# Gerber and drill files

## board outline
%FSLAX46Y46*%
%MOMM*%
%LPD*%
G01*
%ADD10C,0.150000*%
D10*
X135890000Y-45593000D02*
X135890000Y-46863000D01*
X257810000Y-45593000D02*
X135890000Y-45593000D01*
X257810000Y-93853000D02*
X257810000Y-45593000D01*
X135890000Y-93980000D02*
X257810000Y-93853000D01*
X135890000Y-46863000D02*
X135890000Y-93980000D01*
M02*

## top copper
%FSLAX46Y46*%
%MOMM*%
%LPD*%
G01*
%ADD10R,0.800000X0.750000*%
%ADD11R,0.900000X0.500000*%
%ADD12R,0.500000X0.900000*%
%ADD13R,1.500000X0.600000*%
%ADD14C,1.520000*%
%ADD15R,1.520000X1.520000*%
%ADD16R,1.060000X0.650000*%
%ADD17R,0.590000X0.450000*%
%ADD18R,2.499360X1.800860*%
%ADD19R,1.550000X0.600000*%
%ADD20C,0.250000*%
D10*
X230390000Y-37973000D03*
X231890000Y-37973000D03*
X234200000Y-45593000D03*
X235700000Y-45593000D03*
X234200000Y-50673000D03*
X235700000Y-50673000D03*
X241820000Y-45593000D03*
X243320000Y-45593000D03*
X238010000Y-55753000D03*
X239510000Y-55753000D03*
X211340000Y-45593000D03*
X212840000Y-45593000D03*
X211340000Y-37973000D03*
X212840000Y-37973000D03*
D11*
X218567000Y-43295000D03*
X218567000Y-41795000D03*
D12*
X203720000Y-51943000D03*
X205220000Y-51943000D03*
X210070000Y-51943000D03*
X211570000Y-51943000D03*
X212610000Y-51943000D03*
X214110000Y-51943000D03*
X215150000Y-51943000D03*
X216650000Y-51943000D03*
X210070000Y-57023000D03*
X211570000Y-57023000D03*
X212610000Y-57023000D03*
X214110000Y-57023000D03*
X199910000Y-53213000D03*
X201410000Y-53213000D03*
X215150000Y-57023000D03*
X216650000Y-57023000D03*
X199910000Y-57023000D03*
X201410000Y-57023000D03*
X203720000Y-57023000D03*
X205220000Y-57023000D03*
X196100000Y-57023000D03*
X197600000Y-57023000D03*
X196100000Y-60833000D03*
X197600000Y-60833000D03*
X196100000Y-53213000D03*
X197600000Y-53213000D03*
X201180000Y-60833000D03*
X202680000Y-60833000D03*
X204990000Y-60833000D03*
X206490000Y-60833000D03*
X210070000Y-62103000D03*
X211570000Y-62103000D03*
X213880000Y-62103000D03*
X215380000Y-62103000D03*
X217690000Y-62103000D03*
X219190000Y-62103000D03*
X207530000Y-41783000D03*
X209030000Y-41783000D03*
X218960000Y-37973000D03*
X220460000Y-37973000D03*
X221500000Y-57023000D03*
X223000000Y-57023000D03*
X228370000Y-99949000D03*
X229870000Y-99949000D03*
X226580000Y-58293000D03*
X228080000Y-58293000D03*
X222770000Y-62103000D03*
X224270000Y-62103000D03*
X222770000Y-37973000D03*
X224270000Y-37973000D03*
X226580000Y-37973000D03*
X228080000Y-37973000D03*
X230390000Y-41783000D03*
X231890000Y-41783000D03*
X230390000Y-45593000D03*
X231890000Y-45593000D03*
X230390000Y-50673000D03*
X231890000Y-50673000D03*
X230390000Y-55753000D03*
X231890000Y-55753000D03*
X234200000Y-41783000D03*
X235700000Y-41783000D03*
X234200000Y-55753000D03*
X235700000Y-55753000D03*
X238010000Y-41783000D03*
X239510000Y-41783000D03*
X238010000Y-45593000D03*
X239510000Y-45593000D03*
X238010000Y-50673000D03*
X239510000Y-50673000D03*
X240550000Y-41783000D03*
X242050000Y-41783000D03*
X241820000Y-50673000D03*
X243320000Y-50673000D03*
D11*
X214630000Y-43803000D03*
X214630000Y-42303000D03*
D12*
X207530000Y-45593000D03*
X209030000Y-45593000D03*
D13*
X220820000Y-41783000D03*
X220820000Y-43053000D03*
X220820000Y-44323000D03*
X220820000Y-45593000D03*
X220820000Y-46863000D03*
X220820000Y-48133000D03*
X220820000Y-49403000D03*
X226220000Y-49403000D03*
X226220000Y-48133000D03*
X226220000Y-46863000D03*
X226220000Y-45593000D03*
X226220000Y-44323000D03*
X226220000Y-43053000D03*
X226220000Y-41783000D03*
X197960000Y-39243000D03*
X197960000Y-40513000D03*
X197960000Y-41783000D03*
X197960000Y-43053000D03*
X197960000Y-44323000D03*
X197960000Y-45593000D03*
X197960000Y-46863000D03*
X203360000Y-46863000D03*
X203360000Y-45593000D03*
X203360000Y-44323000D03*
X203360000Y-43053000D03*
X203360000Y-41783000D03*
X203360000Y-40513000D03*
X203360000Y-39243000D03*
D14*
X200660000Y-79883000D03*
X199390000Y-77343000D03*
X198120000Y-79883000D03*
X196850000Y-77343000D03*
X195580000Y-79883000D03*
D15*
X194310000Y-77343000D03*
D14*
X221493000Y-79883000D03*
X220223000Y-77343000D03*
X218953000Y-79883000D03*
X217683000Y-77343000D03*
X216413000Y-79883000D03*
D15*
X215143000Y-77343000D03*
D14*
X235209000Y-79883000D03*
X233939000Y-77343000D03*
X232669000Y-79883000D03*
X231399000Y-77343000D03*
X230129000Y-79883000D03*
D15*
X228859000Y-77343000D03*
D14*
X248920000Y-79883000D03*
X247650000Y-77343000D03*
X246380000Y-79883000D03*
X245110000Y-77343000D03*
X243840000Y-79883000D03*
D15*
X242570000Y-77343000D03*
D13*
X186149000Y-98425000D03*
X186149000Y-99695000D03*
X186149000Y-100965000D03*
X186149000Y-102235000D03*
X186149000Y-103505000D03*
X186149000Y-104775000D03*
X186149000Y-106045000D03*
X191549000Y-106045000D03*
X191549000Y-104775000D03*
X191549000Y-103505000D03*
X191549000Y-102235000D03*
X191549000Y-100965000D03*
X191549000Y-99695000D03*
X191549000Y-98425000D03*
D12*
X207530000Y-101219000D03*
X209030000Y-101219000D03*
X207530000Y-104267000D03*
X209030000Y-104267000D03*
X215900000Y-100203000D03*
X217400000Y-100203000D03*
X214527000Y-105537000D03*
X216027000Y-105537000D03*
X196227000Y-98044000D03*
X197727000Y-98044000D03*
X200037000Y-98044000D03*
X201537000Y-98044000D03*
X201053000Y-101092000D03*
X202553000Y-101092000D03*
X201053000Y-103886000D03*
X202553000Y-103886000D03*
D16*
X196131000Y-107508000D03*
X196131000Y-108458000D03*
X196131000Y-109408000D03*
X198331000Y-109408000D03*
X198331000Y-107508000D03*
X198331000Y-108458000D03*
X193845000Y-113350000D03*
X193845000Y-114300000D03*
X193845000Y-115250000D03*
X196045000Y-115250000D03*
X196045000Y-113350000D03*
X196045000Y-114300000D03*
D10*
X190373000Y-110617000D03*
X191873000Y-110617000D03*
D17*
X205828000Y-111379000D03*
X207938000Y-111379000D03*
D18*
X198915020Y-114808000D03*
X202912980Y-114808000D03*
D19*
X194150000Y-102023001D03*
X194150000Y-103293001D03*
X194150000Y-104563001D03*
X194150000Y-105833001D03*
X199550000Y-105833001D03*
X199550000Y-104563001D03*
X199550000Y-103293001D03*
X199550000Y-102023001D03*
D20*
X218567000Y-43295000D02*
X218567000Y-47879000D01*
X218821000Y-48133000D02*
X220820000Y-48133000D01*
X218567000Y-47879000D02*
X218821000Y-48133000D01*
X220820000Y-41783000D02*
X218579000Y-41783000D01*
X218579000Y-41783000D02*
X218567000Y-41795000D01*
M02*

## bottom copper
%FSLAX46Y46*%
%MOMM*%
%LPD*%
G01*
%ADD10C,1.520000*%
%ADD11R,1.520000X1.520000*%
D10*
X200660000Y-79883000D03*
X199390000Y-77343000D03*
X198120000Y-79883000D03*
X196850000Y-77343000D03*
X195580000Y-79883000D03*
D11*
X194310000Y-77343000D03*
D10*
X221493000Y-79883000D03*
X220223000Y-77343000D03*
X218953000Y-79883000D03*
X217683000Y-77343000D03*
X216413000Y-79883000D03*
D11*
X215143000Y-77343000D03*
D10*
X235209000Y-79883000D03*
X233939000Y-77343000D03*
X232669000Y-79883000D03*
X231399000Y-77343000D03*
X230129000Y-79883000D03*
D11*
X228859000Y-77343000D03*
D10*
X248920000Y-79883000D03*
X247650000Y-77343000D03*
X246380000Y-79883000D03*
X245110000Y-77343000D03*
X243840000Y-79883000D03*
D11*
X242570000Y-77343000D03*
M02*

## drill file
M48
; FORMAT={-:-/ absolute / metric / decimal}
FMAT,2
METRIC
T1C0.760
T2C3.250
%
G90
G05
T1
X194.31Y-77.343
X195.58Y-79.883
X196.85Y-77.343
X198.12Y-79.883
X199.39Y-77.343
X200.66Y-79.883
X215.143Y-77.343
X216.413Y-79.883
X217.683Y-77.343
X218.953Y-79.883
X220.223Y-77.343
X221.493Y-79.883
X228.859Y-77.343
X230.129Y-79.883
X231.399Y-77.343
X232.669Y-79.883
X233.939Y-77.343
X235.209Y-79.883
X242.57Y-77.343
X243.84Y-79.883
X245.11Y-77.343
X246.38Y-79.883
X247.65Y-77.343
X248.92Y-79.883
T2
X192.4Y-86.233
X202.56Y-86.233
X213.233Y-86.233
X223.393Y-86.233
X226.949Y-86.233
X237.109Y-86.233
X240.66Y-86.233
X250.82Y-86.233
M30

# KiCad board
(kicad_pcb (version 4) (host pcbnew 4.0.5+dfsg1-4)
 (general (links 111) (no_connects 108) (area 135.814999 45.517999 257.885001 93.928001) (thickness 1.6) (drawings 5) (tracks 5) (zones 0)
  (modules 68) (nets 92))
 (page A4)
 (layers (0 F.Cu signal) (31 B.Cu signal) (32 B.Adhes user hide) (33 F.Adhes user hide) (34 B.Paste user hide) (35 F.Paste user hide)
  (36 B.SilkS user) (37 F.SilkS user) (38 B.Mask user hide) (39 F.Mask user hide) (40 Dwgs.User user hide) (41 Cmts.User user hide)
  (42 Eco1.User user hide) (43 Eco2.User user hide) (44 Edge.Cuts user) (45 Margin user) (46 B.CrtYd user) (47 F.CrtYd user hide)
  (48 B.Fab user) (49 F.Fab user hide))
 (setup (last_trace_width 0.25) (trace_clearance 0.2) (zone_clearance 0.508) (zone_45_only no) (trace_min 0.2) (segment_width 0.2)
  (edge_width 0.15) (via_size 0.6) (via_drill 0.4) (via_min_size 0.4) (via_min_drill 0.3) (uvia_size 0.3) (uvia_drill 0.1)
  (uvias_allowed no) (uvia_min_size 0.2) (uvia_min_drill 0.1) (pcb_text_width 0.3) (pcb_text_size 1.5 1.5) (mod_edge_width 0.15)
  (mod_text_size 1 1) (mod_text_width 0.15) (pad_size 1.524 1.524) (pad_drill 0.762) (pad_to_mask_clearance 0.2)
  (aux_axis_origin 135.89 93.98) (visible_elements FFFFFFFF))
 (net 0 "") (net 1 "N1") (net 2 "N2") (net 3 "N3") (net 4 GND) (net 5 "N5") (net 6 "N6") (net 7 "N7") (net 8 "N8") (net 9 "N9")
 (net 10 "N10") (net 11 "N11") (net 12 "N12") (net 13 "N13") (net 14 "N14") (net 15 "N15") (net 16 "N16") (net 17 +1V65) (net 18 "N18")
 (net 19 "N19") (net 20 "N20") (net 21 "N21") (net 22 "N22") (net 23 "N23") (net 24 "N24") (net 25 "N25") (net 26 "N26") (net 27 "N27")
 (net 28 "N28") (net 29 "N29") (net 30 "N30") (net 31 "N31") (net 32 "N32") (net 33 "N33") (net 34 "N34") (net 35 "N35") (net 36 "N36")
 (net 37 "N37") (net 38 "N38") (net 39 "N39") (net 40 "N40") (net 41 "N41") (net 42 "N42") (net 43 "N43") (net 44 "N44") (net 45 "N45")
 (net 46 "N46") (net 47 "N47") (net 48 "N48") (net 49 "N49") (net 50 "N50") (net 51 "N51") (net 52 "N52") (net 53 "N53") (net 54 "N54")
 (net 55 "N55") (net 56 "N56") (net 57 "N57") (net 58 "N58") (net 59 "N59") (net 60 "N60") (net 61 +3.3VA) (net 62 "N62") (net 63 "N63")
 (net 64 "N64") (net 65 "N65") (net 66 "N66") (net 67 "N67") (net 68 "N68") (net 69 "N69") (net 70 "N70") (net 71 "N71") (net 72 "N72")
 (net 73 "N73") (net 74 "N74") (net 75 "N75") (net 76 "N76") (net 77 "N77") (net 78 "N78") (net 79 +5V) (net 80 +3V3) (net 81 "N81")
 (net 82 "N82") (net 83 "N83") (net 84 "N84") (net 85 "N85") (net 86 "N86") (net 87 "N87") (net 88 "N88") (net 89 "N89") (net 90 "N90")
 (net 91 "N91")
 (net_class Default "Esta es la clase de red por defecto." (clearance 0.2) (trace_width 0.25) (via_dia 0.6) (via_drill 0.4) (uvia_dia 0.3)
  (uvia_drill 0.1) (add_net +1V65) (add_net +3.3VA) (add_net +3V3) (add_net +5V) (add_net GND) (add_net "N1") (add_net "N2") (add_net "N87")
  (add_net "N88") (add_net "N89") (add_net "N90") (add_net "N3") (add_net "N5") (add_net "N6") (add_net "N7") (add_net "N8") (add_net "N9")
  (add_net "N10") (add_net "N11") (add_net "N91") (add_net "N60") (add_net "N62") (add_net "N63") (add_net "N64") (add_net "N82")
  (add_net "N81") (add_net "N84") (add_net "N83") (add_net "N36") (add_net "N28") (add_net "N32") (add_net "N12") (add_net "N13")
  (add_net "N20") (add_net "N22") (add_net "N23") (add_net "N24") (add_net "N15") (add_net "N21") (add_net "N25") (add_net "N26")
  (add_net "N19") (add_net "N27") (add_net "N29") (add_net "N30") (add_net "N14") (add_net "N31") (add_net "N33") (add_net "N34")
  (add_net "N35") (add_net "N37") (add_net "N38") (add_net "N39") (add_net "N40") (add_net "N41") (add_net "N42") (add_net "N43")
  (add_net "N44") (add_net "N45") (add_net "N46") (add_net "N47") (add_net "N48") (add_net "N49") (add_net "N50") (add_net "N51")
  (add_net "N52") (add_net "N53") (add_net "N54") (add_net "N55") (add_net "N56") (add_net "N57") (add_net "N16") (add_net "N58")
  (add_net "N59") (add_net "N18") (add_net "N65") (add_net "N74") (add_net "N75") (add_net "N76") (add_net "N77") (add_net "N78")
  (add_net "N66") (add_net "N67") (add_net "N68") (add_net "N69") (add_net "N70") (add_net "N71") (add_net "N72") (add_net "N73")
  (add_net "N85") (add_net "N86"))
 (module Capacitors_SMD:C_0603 (layer F.Cu) (at 231.14 37.973)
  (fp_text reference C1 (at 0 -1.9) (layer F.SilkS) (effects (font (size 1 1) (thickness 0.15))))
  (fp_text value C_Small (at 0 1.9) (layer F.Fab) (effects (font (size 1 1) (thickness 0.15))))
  (pad 1 smd rect (at -0.75 0) (size 0.8 0.75) (layers F.Cu F.Paste F.Mask) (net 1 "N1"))
  (pad 2 smd rect (at 0.75 0) (size 0.8 0.75) (layers F.Cu F.Paste F.Mask) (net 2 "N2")))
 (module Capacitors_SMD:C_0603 (layer F.Cu) (at 234.95 45.593)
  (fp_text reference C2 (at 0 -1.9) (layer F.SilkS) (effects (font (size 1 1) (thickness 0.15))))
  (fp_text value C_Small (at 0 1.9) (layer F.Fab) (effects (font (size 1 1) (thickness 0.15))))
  (pad 1 smd rect (at -0.75 0) (size 0.8 0.75) (layers F.Cu F.Paste F.Mask) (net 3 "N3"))
  (pad 2 smd rect (at 0.75 0) (size 0.8 0.75) (layers F.Cu F.Paste F.Mask) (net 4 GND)))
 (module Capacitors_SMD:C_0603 (layer F.Cu) (at 234.95 50.673)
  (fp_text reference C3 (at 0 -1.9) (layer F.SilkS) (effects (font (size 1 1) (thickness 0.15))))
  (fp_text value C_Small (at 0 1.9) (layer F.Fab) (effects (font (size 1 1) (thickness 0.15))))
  (pad 1 smd rect (at -0.75 0) (size 0.8 0.75) (layers F.Cu F.Paste F.Mask) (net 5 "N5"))
  (pad 2 smd rect (at 0.75 0) (size 0.8 0.75) (layers F.Cu F.Paste F.Mask) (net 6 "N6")))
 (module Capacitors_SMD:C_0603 (layer F.Cu) (at 242.57 45.593)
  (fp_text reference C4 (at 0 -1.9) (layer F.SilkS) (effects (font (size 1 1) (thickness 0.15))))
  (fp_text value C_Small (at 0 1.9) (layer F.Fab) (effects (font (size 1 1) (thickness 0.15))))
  (pad 1 smd rect (at -0.75 0) (size 0.8 0.75) (layers F.Cu F.Paste F.Mask) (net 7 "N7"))
  (pad 2 smd rect (at 0.75 0) (size 0.8 0.75) (layers F.Cu F.Paste F.Mask) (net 4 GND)))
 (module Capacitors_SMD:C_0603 (layer F.Cu) (at 238.76 55.753)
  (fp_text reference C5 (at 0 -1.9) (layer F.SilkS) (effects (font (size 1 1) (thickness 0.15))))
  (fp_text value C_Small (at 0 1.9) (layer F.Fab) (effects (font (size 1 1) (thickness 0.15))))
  (pad 1 smd rect (at -0.75 0) (size 0.8 0.75) (layers F.Cu F.Paste F.Mask) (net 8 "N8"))
  (pad 2 smd rect (at 0.75 0) (size 0.8 0.75) (layers F.Cu F.Paste F.Mask) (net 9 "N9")))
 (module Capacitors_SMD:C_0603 (layer F.Cu) (at 212.09 45.593)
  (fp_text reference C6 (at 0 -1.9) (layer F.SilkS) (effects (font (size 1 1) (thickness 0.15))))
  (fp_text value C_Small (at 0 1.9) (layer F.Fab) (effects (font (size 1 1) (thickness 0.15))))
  (pad 1 smd rect (at -0.75 0) (size 0.8 0.75) (layers F.Cu F.Paste F.Mask) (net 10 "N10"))
  (pad 2 smd rect (at 0.75 0) (size 0.8 0.75) (layers F.Cu F.Paste F.Mask) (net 4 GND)))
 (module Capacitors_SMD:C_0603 (layer F.Cu) (at 212.09 37.973)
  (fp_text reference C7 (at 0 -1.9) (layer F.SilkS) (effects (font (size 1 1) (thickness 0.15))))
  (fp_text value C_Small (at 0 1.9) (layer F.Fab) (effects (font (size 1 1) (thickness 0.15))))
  (pad 1 smd rect (at -0.75 0) (size 0.8 0.75) (layers F.Cu F.Paste F.Mask) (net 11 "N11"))
  (pad 2 smd rect (at 0.75 0) (size 0.8 0.75) (layers F.Cu F.Paste F.Mask) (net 4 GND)))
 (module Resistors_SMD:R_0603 (layer F.Cu) (at 218.567 42.545 90)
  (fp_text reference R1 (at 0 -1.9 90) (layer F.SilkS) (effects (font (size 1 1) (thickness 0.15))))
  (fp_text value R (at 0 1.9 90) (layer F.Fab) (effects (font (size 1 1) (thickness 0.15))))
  (pad 1 smd rect (at -0.75 0 90) (size 0.5 0.9) (layers F.Cu F.Paste F.Mask) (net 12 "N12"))
  (pad 2 smd rect (at 0.75 0 90) (size 0.5 0.9) (layers F.Cu F.Paste F.Mask) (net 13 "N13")))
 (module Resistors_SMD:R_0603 (layer F.Cu) (at 204.47 51.943)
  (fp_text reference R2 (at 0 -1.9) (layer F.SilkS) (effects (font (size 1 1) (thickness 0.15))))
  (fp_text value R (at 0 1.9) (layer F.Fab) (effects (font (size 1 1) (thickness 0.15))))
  (pad 1 smd rect (at -0.75 0) (size 0.5 0.9) (layers F.Cu F.Paste F.Mask) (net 13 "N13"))
  (pad 2 smd rect (at 0.75 0) (size 0.5 0.9) (layers F.Cu F.Paste F.Mask) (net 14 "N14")))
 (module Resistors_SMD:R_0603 (layer F.Cu) (at 210.82 51.943)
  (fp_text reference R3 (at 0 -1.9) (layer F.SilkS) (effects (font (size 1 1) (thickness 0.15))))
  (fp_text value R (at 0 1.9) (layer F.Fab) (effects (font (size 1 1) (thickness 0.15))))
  (pad 1 smd rect (at -0.75 0) (size 0.5 0.9) (layers F.Cu F.Paste F.Mask) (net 7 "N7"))
  (pad 2 smd rect (at 0.75 0) (size 0.5 0.9) (layers F.Cu F.Paste F.Mask) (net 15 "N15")))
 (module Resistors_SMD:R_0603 (layer F.Cu) (at 213.36 51.943)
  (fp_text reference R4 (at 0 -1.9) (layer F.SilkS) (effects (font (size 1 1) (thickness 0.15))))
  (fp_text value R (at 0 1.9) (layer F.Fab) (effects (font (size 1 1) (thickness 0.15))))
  (pad 1 smd rect (at -0.75 0) (size 0.5 0.9) (layers F.Cu F.Paste F.Mask) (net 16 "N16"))
  (pad 2 smd rect (at 0.75 0) (size 0.5 0.9) (layers F.Cu F.Paste F.Mask) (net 12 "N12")))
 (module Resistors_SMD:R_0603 (layer F.Cu) (at 215.9 51.943)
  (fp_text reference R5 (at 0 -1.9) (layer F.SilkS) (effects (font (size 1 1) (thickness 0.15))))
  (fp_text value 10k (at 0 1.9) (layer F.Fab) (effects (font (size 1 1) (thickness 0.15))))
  (pad 1 smd rect (at -0.75 0) (size 0.5 0.9) (layers F.Cu F.Paste F.Mask) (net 14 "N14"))
  (pad 2 smd rect (at 0.75 0) (size 0.5 0.9) (layers F.Cu F.Paste F.Mask) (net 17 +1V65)))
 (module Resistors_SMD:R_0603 (layer F.Cu) (at 210.82 57.023)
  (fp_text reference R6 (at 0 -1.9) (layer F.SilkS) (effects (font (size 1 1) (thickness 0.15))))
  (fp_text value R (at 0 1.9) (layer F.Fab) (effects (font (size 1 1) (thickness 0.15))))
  (pad 1 smd rect (at -0.75 0) (size 0.5 0.9) (layers F.Cu F.Paste F.Mask) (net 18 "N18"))
  (pad 2 smd rect (at 0.75 0) (size 0.5 0.9) (layers F.Cu F.Paste F.Mask) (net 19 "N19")))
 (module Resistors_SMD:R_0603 (layer F.Cu) (at 213.36 57.023)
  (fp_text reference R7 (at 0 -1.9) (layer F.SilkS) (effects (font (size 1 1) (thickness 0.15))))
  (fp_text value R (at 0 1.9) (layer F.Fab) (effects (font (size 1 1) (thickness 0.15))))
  (pad 1 smd rect (at -0.75 0) (size 0.5 0.9) (layers F.Cu F.Paste F.Mask) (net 3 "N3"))
  (pad 2 smd rect (at 0.75 0) (size 0.5 0.9) (layers F.Cu F.Paste F.Mask) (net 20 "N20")))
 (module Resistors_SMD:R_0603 (layer F.Cu) (at 200.66 53.213)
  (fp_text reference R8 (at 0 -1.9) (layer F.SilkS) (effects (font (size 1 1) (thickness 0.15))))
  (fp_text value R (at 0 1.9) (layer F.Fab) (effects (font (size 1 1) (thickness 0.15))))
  (pad 1 smd rect (at -0.75 0) (size 0.5 0.9) (layers F.Cu F.Paste F.Mask) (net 10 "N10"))
  (pad 2 smd rect (at 0.75 0) (size 0.5 0.9) (layers F.Cu F.Paste F.Mask) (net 16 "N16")))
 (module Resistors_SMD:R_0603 (layer F.Cu) (at 215.9 57.023)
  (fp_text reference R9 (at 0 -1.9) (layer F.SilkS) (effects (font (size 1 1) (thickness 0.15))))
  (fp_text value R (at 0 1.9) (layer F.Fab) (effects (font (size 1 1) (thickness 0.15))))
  (pad 1 smd rect (at -0.75 0) (size 0.5 0.9) (layers F.Cu F.Paste F.Mask) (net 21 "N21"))
  (pad 2 smd rect (at 0.75 0) (size 0.5 0.9) (layers F.Cu F.Paste F.Mask) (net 18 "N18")))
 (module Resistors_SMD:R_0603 (layer F.Cu) (at 200.66 57.023)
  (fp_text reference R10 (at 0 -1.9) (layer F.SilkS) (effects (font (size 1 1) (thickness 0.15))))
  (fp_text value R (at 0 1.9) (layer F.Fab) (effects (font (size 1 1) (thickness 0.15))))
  (pad 1 smd rect (at -0.75 0) (size 0.5 0.9) (layers F.Cu F.Paste F.Mask) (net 20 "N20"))
  (pad 2 smd rect (at 0.75 0) (size 0.5 0.9) (layers F.Cu F.Paste F.Mask) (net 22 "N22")))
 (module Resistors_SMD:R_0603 (layer F.Cu) (at 204.47 57.023)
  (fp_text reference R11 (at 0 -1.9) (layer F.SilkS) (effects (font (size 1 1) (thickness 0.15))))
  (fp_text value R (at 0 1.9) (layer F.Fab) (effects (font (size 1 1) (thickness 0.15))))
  (pad 1 smd rect (at -0.75 0) (size 0.5 0.9) (layers F.Cu F.Paste F.Mask) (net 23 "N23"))
  (pad 2 smd rect (at 0.75 0) (size 0.5 0.9) (layers F.Cu F.Paste F.Mask) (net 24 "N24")))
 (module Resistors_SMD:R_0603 (layer F.Cu) (at 196.85 57.023)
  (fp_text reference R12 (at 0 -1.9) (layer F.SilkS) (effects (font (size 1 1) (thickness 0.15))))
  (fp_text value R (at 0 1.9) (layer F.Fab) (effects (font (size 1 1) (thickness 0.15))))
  (pad 1 smd rect (at -0.75 0) (size 0.5 0.9) (layers F.Cu F.Paste F.Mask) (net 15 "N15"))
  (pad 2 smd rect (at 0.75 0) (size 0.5 0.9) (layers F.Cu F.Paste F.Mask) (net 21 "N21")))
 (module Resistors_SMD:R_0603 (layer F.Cu) (at 196.85 60.833)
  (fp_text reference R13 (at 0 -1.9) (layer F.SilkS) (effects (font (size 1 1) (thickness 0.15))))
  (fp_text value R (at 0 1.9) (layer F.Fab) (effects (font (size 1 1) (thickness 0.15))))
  (pad 1 smd rect (at -0.75 0) (size 0.5 0.9) (layers F.Cu F.Paste F.Mask) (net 22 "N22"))
  (pad 2 smd rect (at 0.75 0) (size 0.5 0.9) (layers F.Cu F.Paste F.Mask) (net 23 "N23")))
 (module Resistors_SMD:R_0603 (layer F.Cu) (at 196.85 53.213)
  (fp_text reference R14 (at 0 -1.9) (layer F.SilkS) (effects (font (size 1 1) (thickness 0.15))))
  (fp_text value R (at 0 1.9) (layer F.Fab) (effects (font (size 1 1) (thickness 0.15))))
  (pad 1 smd rect (at -0.75 0) (size 0.5 0.9) (layers F.Cu F.Paste F.Mask) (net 11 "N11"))
  (pad 2 smd rect (at 0.75 0) (size 0.5 0.9) (layers F.Cu F.Paste F.Mask) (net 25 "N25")))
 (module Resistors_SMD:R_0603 (layer F.Cu) (at 201.93 60.833)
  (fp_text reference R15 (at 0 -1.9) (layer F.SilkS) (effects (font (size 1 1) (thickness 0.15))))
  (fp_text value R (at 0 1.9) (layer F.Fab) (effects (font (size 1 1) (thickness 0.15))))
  (pad 1 smd rect (at -0.75 0) (size 0.5 0.9) (layers F.Cu F.Paste F.Mask) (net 25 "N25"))
  (pad 2 smd rect (at 0.75 0) (size 0.5 0.9) (layers F.Cu F.Paste F.Mask) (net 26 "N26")))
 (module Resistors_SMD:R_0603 (layer F.Cu) (at 205.74 60.833)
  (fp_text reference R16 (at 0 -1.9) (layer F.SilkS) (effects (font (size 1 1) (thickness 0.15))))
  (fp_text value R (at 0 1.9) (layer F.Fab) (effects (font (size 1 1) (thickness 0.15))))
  (pad 1 smd rect (at -0.75 0) (size 0.5 0.9) (layers F.Cu F.Paste F.Mask) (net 19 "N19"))
  (pad 2 smd rect (at 0.75 0) (size 0.5 0.9) (layers F.Cu F.Paste F.Mask) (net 17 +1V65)))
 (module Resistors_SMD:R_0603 (layer F.Cu) (at 210.82 62.103)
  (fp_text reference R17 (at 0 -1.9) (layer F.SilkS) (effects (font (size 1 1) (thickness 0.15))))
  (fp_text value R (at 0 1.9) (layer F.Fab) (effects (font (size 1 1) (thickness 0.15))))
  (pad 1 smd rect (at -0.75 0) (size 0.5 0.9) (layers F.Cu F.Paste F.Mask) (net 24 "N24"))
  (pad 2 smd rect (at 0.75 0) (size 0.5 0.9) (layers F.Cu F.Paste F.Mask) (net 17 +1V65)))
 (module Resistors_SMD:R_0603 (layer F.Cu) (at 214.63 62.103)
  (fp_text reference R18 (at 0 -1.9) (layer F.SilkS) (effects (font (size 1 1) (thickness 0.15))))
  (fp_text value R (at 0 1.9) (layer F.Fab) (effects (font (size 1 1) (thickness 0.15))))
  (pad 1 smd rect (at -0.75 0) (size 0.5 0.9) (layers F.Cu F.Paste F.Mask) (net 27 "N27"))
  (pad 2 smd rect (at 0.75 0) (size 0.5 0.9) (layers F.Cu F.Paste F.Mask) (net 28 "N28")))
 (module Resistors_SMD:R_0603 (layer F.Cu) (at 218.44 62.103)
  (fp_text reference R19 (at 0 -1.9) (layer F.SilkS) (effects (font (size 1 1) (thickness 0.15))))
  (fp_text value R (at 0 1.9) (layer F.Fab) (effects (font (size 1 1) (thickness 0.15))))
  (pad 1 smd rect (at -0.75 0) (size 0.5 0.9) (layers F.Cu F.Paste F.Mask) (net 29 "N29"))
  (pad 2 smd rect (at 0.75 0) (size 0.5 0.9) (layers F.Cu F.Paste F.Mask) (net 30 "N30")))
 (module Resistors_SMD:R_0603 (layer F.Cu) (at 208.28 41.783)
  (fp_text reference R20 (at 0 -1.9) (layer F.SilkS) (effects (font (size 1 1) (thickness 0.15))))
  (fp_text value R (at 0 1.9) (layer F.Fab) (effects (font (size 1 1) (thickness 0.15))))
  (pad 1 smd rect (at -0.75 0) (size 0.5 0.9) (layers F.Cu F.Paste F.Mask) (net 26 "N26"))
  (pad 2 smd rect (at 0.75 0) (size 0.5 0.9) (layers F.Cu F.Paste F.Mask) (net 29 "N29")))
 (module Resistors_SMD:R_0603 (layer F.Cu) (at 219.71 37.973)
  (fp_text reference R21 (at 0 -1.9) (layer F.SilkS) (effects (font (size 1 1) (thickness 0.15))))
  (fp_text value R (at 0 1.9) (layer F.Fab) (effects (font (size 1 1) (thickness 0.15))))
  (pad 1 smd rect (at -0.75 0) (size 0.5 0.9) (layers F.Cu F.Paste F.Mask) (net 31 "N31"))
  (pad 2 smd rect (at 0.75 0) (size 0.5 0.9) (layers F.Cu F.Paste F.Mask) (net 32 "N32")))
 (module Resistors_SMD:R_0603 (layer F.Cu) (at 222.25 57.023)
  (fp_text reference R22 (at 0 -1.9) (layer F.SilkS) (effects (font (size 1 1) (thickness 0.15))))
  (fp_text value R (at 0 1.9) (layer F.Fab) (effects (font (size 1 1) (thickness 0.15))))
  (pad 1 smd rect (at -0.75 0) (size 0.5 0.9) (layers F.Cu F.Paste F.Mask) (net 30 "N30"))
  (pad 2 smd rect (at 0.75 0) (size 0.5 0.9) (layers F.Cu F.Paste F.Mask) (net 17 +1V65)))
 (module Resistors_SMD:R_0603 (layer F.Cu) (at 229.12 99.949)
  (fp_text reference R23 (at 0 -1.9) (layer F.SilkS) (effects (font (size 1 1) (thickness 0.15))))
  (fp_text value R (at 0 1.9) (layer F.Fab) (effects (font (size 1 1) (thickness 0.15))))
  (pad 1 smd rect (at -0.75 0) (size 0.5 0.9) (layers F.Cu F.Paste F.Mask) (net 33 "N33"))
  (pad 2 smd rect (at 0.75 0) (size 0.5 0.9) (layers F.Cu F.Paste F.Mask) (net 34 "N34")))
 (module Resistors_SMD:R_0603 (layer F.Cu) (at 227.33 58.293)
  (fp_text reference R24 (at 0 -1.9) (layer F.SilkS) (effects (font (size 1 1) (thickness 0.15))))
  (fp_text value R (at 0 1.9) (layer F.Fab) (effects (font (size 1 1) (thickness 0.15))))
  (pad 1 smd rect (at -0.75 0) (size 0.5 0.9) (layers F.Cu F.Paste F.Mask) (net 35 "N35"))
  (pad 2 smd rect (at 0.75 0) (size 0.5 0.9) (layers F.Cu F.Paste F.Mask) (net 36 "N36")))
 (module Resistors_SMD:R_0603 (layer F.Cu) (at 223.52 62.103)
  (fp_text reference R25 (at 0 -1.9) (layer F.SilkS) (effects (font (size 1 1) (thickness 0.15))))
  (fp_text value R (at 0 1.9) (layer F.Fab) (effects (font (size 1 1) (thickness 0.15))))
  (pad 1 smd rect (at -0.75 0) (size 0.5 0.9) (layers F.Cu F.Paste F.Mask) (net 35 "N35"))
  (pad 2 smd rect (at 0.75 0) (size 0.5 0.9) (layers F.Cu F.Paste F.Mask) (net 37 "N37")))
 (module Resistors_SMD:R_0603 (layer F.Cu) (at 223.52 37.973)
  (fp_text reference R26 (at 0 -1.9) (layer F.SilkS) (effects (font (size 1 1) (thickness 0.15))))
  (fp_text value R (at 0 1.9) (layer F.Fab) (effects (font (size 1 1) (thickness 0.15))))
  (pad 1 smd rect (at -0.75 0) (size 0.5 0.9) (layers F.Cu F.Paste F.Mask) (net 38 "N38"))
  (pad 2 smd rect (at 0.75 0) (size 0.5 0.9) (layers F.Cu F.Paste F.Mask) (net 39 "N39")))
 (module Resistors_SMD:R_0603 (layer F.Cu) (at 227.33 37.973)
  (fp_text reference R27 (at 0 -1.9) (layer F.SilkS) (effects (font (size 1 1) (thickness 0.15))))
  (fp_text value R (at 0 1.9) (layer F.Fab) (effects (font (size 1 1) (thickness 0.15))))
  (pad 1 smd rect (at -0.75 0) (size 0.5 0.9) (layers F.Cu F.Paste F.Mask) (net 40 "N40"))
  (pad 2 smd rect (at 0.75 0) (size 0.5 0.9) (layers F.Cu F.Paste F.Mask) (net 27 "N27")))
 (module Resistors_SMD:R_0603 (layer F.Cu) (at 231.14 41.783)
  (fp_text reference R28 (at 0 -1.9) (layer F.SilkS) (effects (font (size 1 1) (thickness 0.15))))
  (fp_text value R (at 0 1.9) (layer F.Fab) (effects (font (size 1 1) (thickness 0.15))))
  (pad 1 smd rect (at -0.75 0) (size 0.5 0.9) (layers F.Cu F.Paste F.Mask) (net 39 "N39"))
  (pad 2 smd rect (at 0.75 0) (size 0.5 0.9) (layers F.Cu F.Paste F.Mask) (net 31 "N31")))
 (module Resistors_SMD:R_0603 (layer F.Cu) (at 231.14 45.593)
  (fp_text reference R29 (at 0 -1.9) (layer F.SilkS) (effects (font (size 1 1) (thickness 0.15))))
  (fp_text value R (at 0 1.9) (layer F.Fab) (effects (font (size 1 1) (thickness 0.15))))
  (pad 1 smd rect (at -0.75 0) (size 0.5 0.9) (layers F.Cu F.Paste F.Mask) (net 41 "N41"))
  (pad 2 smd rect (at 0.75 0) (size 0.5 0.9) (layers F.Cu F.Paste F.Mask) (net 37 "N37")))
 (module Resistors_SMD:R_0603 (layer F.Cu) (at 231.14 50.673)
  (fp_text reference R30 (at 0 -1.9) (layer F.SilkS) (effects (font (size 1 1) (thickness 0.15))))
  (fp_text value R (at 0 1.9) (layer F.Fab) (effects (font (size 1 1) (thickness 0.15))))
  (pad 1 smd rect (at -0.75 0) (size 0.5 0.9) (layers F.Cu F.Paste F.Mask) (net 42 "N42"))
  (pad 2 smd rect (at 0.75 0) (size 0.5 0.9) (layers F.Cu F.Paste F.Mask) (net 40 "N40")))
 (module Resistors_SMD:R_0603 (layer F.Cu) (at 231.14 55.753)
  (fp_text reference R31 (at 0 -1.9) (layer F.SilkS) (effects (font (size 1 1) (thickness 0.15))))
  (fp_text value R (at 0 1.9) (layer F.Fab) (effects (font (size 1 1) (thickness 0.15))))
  (pad 1 smd rect (at -0.75 0) (size 0.5 0.9) (layers F.Cu F.Paste F.Mask) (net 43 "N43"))
  (pad 2 smd rect (at 0.75 0) (size 0.5 0.9) (layers F.Cu F.Paste F.Mask) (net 41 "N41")))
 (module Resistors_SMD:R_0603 (layer F.Cu) (at 234.95 41.783)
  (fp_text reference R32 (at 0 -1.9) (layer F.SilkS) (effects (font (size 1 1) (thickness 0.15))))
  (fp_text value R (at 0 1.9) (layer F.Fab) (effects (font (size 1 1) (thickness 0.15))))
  (pad 1 smd rect (at -0.75 0) (size 0.5 0.9) (layers F.Cu F.Paste F.Mask) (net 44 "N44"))
  (pad 2 smd rect (at 0.75 0) (size 0.5 0.9) (layers F.Cu F.Paste F.Mask) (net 42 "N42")))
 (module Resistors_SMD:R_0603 (layer F.Cu) (at 234.95 55.753)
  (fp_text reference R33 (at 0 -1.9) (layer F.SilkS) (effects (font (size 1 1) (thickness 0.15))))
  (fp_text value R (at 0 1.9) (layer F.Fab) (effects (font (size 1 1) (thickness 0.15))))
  (pad 1 smd rect (at -0.75 0) (size 0.5 0.9) (layers F.Cu F.Paste F.Mask) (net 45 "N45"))
  (pad 2 smd rect (at 0.75 0) (size 0.5 0.9) (layers F.Cu F.Paste F.Mask) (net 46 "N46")))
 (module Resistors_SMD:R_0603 (layer F.Cu) (at 238.76 41.783)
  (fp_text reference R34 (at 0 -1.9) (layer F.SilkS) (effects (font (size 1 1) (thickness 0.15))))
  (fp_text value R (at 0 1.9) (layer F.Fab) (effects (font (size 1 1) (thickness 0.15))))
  (pad 1 smd rect (at -0.75 0) (size 0.5 0.9) (layers F.Cu F.Paste F.Mask) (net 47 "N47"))
  (pad 2 smd rect (at 0.75 0) (size 0.5 0.9) (layers F.Cu F.Paste F.Mask) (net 38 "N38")))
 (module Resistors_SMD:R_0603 (layer F.Cu) (at 238.76 45.593)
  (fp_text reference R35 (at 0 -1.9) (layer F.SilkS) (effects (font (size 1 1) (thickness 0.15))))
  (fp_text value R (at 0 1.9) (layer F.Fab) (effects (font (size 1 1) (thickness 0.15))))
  (pad 1 smd rect (at -0.75 0) (size 0.5 0.9) (layers F.Cu F.Paste F.Mask) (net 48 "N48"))
  (pad 2 smd rect (at 0.75 0) (size 0.5 0.9) (layers F.Cu F.Paste F.Mask) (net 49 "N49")))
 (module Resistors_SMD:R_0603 (layer F.Cu) (at 238.76 50.673)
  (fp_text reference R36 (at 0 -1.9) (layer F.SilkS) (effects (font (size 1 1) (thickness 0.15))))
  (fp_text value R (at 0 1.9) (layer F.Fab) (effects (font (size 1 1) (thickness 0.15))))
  (pad 1 smd rect (at -0.75 0) (size 0.5 0.9) (layers F.Cu F.Paste F.Mask) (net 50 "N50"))
  (pad 2 smd rect (at 0.75 0) (size 0.5 0.9) (layers F.Cu F.Paste F.Mask) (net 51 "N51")))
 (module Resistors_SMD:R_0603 (layer F.Cu) (at 241.3 41.783)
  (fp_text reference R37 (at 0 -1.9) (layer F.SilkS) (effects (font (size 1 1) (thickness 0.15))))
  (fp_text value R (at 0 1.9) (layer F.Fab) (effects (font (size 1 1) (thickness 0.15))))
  (pad 1 smd rect (at -0.75 0) (size 0.5 0.9) (layers F.Cu F.Paste F.Mask) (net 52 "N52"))
  (pad 2 smd rect (at 0.75 0) (size 0.5 0.9) (layers F.Cu F.Paste F.Mask) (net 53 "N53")))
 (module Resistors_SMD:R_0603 (layer F.Cu) (at 242.57 50.673)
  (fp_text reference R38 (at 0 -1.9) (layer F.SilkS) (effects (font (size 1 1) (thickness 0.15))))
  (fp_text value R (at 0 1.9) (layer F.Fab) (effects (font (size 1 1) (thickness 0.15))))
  (pad 1 smd rect (at -0.75 0) (size 0.5 0.9) (layers F.Cu F.Paste F.Mask) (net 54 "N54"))
  (pad 2 smd rect (at 0.75 0) (size 0.5 0.9) (layers F.Cu F.Paste F.Mask) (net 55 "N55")))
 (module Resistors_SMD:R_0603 (layer F.Cu) (at 214.63 43.053 90)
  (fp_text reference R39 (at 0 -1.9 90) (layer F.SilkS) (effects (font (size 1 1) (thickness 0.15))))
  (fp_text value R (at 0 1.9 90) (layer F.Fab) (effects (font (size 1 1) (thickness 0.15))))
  (pad 1 smd rect (at -0.75 0 90) (size 0.5 0.9) (layers F.Cu F.Paste F.Mask) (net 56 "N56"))
  (pad 2 smd rect (at 0.75 0 90) (size 0.5 0.9) (layers F.Cu F.Paste F.Mask) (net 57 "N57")))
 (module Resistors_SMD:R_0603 (layer F.Cu) (at 208.28 45.593)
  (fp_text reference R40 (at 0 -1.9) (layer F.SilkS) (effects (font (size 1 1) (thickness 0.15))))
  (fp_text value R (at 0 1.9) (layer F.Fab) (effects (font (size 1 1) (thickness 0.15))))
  (pad 1 smd rect (at -0.75 0) (size 0.5 0.9) (layers F.Cu F.Paste F.Mask) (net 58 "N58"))
  (pad 2 smd rect (at 0.75 0) (size 0.5 0.9) (layers F.Cu F.Paste F.Mask) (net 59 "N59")))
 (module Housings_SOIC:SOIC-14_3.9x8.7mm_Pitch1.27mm (layer F.Cu) (at 223.52 45.593)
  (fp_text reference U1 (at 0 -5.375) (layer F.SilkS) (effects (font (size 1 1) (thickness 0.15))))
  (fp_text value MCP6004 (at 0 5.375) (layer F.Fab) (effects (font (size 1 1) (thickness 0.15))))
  (pad 1 smd rect (at -2.7 -3.81) (size 1.5 0.6) (layers F.Cu F.Paste F.Mask) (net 13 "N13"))
  (pad 2 smd rect (at -2.7 -2.54) (size 1.5 0.6) (layers F.Cu F.Paste F.Mask) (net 14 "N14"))
  (pad 3 smd rect (at -2.7 -1.27) (size 1.5 0.6) (layers F.Cu F.Paste F.Mask) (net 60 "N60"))
  (pad 4 smd rect (at -2.7 0) (size 1.5 0.6) (layers F.Cu F.Paste F.Mask) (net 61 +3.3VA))
  (pad 5 smd rect (at -2.7 1.27) (size 1.5 0.6) (layers F.Cu F.Paste F.Mask) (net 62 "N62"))
  (pad 6 smd rect (at -2.7 2.54) (size 1.5 0.6) (layers F.Cu F.Paste F.Mask) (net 12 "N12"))
  (pad 7 smd rect (at -2.7 3.81) (size 1.5 0.6) (layers F.Cu F.Paste F.Mask) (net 16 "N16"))
  (pad 8 smd rect (at 2.7 3.81) (size 1.5 0.6) (layers F.Cu F.Paste F.Mask) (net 18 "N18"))
  (pad 9 smd rect (at 2.7 2.54) (size 1.5 0.6) (layers F.Cu F.Paste F.Mask) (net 19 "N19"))
  (pad 10 smd rect (at 2.7 1.27) (size 1.5 0.6) (layers F.Cu F.Paste F.Mask) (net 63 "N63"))
  (pad 11 smd rect (at 2.7 0) (size 1.5 0.6) (layers F.Cu F.Paste F.Mask) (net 4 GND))
  (pad 12 smd rect (at 2.7 -1.27) (size 1.5 0.6) (layers F.Cu F.Paste F.Mask) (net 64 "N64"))
  (pad 13 smd rect (at 2.7 -2.54) (size 1.5 0.6) (layers F.Cu F.Paste F.Mask) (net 21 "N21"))
  (pad 14 smd rect (at 2.7 -3.81) (size 1.5 0.6) (layers F.Cu F.Paste F.Mask) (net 15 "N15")))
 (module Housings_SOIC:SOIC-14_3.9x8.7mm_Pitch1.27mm (layer F.Cu) (at 200.66 43.053)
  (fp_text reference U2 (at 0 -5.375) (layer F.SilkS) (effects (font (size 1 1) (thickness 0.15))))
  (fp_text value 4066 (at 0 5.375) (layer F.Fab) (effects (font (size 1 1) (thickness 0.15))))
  (pad 1 smd rect (at -2.7 -3.81) (size 1.5 0.6) (layers F.Cu F.Paste F.Mask) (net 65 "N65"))
  (pad 2 smd rect (at -2.7 -2.54) (size 1.5 0.6) (layers F.Cu F.Paste F.Mask) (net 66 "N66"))
  (pad 3 smd rect (at -2.7 -1.27) (size 1.5 0.6) (layers F.Cu F.Paste F.Mask) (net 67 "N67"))
  (pad 4 smd rect (at -2.7 0) (size 1.5 0.6) (layers F.Cu F.Paste F.Mask) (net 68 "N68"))
  (pad 5 smd rect (at -2.7 1.27) (size 1.5 0.6) (layers F.Cu F.Paste F.Mask) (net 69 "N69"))
  (pad 6 smd rect (at -2.7 2.54) (size 1.5 0.6) (layers F.Cu F.Paste F.Mask) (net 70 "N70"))
  (pad 7 smd rect (at -2.7 3.81) (size 1.5 0.6) (layers F.Cu F.Paste F.Mask) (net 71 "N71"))
  (pad 8 smd rect (at 2.7 3.81) (size 1.5 0.6) (layers F.Cu F.Paste F.Mask) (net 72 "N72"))
  (pad 9 smd rect (at 2.7 2.54) (size 1.5 0.6) (layers F.Cu F.Paste F.Mask) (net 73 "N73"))
  (pad 10 smd rect (at 2.7 1.27) (size 1.5 0.6) (layers F.Cu F.Paste F.Mask) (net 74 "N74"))
  (pad 11 smd rect (at 2.7 0) (size 1.5 0.6) (layers F.Cu F.Paste F.Mask) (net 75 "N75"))
  (pad 12 smd rect (at 2.7 -1.27) (size 1.5 0.6) (layers F.Cu F.Paste F.Mask) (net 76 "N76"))
  (pad 13 smd rect (at 2.7 -2.54) (size 1.5 0.6) (layers F.Cu F.Paste F.Mask) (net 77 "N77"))
  (pad 14 smd rect (at 2.7 -3.81) (size 1.5 0.6) (layers F.Cu F.Paste F.Mask) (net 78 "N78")))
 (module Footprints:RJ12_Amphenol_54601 (layer F.Cu) (at 194.31 77.343)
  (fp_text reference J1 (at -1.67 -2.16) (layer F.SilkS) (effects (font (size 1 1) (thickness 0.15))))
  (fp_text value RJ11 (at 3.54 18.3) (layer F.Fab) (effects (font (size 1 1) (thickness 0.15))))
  (pad "" np_thru_hole circle (at 8.25 8.89) (size 3.25 3.25) (drill 3.25) (layers *.Cu *.Mask))
  (pad 6 thru_hole circle (at 6.35 2.54) (size 1.52 1.52) (drill 0.76) (layers *.Cu *.Mask) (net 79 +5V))
  (pad 5 thru_hole circle (at 5.08 0) (size 1.52 1.52) (drill 0.76) (layers *.Cu *.Mask) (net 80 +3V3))
  (pad 4 thru_hole circle (at 3.81 2.54) (size 1.52 1.52) (drill 0.76) (layers *.Cu *.Mask) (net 17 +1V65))
  (pad 3 thru_hole circle (at 2.54 0) (size 1.52 1.52) (drill 0.76) (layers *.Cu *.Mask) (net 62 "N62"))
  (pad 2 thru_hole circle (at 1.27 2.54) (size 1.52 1.52) (drill 0.76) (layers *.Cu *.Mask) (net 60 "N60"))
  (pad "" np_thru_hole circle (at -1.91 8.89) (size 3.25 3.25) (drill 3.25) (layers *.Cu *.Mask))
  (pad 1 thru_hole rect (at 0 0) (size 1.52 1.52) (drill 0.76) (layers *.Cu *.Mask) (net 4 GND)))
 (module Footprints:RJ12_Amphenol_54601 (layer F.Cu) (at 215.143 77.343)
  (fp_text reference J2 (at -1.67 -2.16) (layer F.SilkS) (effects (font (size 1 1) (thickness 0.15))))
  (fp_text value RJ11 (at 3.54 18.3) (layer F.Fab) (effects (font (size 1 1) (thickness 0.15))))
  (pad "" np_thru_hole circle (at 8.25 8.89) (size 3.25 3.25) (drill 3.25) (layers *.Cu *.Mask))
  (pad 6 thru_hole circle (at 6.35 2.54) (size 1.52 1.52) (drill 0.76) (layers *.Cu *.Mask) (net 79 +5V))
  (pad 5 thru_hole circle (at 5.08 0) (size 1.52 1.52) (drill 0.76) (layers *.Cu *.Mask) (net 80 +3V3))
  (pad 4 thru_hole circle (at 3.81 2.54) (size 1.52 1.52) (drill 0.76) (layers *.Cu *.Mask) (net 17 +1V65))
  (pad 3 thru_hole circle (at 2.54 0) (size 1.52 1.52) (drill 0.76) (layers *.Cu *.Mask) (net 64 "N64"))
  (pad 2 thru_hole circle (at 1.27 2.54) (size 1.52 1.52) (drill 0.76) (layers *.Cu *.Mask) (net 63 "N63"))
  (pad "" np_thru_hole circle (at -1.91 8.89) (size 3.25 3.25) (drill 3.25) (layers *.Cu *.Mask))
  (pad 1 thru_hole rect (at 0 0) (size 1.52 1.52) (drill 0.76) (layers *.Cu *.Mask) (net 4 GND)))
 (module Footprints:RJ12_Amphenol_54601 (layer F.Cu) (at 228.859 77.343)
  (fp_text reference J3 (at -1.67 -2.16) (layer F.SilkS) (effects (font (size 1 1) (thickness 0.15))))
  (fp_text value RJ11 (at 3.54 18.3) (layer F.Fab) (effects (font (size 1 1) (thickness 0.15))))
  (pad "" np_thru_hole circle (at 8.25 8.89) (size 3.25 3.25) (drill 3.25) (layers *.Cu *.Mask))
  (pad 6 thru_hole circle (at 6.35 2.54) (size 1.52 1.52) (drill 0.76) (layers *.Cu *.Mask) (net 79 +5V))
  (pad 5 thru_hole circle (at 5.08 0) (size 1.52 1.52) (drill 0.76) (layers *.Cu *.Mask) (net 80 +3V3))
  (pad 4 thru_hole circle (at 3.81 2.54) (size 1.52 1.52) (drill 0.76) (layers *.Cu *.Mask) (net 17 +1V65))
  (pad 3 thru_hole circle (at 2.54 0) (size 1.52 1.52) (drill 0.76) (layers *.Cu *.Mask) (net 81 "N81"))
  (pad 2 thru_hole circle (at 1.27 2.54) (size 1.52 1.52) (drill 0.76) (layers *.Cu *.Mask) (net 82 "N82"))
  (pad "" np_thru_hole circle (at -1.91 8.89) (size 3.25 3.25) (drill 3.25) (layers *.Cu *.Mask))
  (pad 1 thru_hole rect (at 0 0) (size 1.52 1.52) (drill 0.76) (layers *.Cu *.Mask) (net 4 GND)))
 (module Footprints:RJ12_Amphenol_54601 (layer F.Cu) (at 242.57 77.343)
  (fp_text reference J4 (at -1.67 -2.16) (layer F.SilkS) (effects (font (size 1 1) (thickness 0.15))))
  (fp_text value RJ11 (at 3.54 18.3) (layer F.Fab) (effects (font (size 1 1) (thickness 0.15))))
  (pad "" np_thru_hole circle (at 8.25 8.89) (size 3.25 3.25) (drill 3.25) (layers *.Cu *.Mask))
  (pad 6 thru_hole circle (at 6.35 2.54) (size 1.52 1.52) (drill 0.76) (layers *.Cu *.Mask) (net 79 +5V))
  (pad 5 thru_hole circle (at 5.08 0) (size 1.52 1.52) (drill 0.76) (layers *.Cu *.Mask) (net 80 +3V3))
  (pad 4 thru_hole circle (at 3.81 2.54) (size 1.52 1.52) (drill 0.76) (layers *.Cu *.Mask) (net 17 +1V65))
  (pad 3 thru_hole circle (at 2.54 0) (size 1.52 1.52) (drill 0.76) (layers *.Cu *.Mask) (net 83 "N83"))
  (pad 2 thru_hole circle (at 1.27 2.54) (size 1.52 1.52) (drill 0.76) (layers *.Cu *.Mask) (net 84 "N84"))
  (pad "" np_thru_hole circle (at -1.91 8.89) (size 3.25 3.25) (drill 3.25) (layers *.Cu *.Mask))
  (pad 1 thru_hole rect (at 0 0) (size 1.52 1.52) (drill 0.76) (layers *.Cu *.Mask) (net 4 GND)))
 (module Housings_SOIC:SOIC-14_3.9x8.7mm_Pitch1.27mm (layer F.Cu) (at 188.849 102.235)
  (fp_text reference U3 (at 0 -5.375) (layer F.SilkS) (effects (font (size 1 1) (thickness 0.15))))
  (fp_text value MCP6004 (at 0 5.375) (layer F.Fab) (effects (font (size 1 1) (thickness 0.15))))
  (pad 1 smd rect (at -2.7 -3.81) (size 1.5 0.6) (layers F.Cu F.Paste F.Mask) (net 29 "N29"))
  (pad 2 smd rect (at -2.7 -2.54) (size 1.5 0.6) (layers F.Cu F.Paste F.Mask) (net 30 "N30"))
  (pad 3 smd rect (at -2.7 -1.27) (size 1.5 0.6) (layers F.Cu F.Paste F.Mask) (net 84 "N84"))
  (pad 4 smd rect (at -2.7 0) (size 1.5 0.6) (layers F.Cu F.Paste F.Mask) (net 61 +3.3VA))
  (pad 5 smd rect (at -2.7 1.27) (size 1.5 0.6) (layers F.Cu F.Paste F.Mask) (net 82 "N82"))
  (pad 6 smd rect (at -2.7 2.54) (size 1.5 0.6) (layers F.Cu F.Paste F.Mask) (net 24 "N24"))
  (pad 7 smd rect (at -2.7 3.81) (size 1.5 0.6) (layers F.Cu F.Paste F.Mask) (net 23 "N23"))
  (pad 8 smd rect (at 2.7 3.81) (size 1.5 0.6) (layers F.Cu F.Paste F.Mask) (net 25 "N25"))
  (pad 9 smd rect (at 2.7 2.54) (size 1.5 0.6) (layers F.Cu F.Paste F.Mask) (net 26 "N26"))
  (pad 10 smd rect (at 2.7 1.27) (size 1.5 0.6) (layers F.Cu F.Paste F.Mask) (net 83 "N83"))
  (pad 11 smd rect (at 2.7 0) (size 1.5 0.6) (layers F.Cu F.Paste F.Mask) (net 4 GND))
  (pad 12 smd rect (at 2.7 -1.27) (size 1.5 0.6) (layers F.Cu F.Paste F.Mask) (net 81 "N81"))
  (pad 13 smd rect (at 2.7 -2.54) (size 1.5 0.6) (layers F.Cu F.Paste F.Mask) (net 22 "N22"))
  (pad 14 smd rect (at 2.7 -3.81) (size 1.5 0.6) (layers F.Cu F.Paste F.Mask) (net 20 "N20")))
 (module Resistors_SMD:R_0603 (layer F.Cu) (at 208.28 101.219)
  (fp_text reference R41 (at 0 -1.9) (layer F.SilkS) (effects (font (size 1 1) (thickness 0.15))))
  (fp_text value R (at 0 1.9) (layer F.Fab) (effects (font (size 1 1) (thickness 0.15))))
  (pad 1 smd rect (at -0.75 0) (size 0.5 0.9) (layers F.Cu F.Paste F.Mask) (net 62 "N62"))
  (pad 2 smd rect (at 0.75 0) (size 0.5 0.9) (layers F.Cu F.Paste F.Mask) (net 60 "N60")))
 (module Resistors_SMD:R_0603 (layer F.Cu) (at 208.28 104.267)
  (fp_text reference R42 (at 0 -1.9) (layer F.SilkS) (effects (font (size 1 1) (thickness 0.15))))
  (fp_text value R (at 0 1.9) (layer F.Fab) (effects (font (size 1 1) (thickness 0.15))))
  (pad 1 smd rect (at -0.75 0) (size 0.5 0.9) (layers F.Cu F.Paste F.Mask) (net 60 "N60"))
  (pad 2 smd rect (at 0.75 0) (size 0.5 0.9) (layers F.Cu F.Paste F.Mask) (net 17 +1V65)))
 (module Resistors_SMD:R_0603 (layer F.Cu) (at 216.65 100.203)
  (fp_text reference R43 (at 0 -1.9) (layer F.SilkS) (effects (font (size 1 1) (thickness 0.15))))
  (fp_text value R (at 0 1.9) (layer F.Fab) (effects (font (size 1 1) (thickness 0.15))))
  (pad 1 smd rect (at -0.75 0) (size 0.5 0.9) (layers F.Cu F.Paste F.Mask) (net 64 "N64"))
  (pad 2 smd rect (at 0.75 0) (size 0.5 0.9) (layers F.Cu F.Paste F.Mask) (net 63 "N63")))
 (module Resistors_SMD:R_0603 (layer F.Cu) (at 215.277 105.537)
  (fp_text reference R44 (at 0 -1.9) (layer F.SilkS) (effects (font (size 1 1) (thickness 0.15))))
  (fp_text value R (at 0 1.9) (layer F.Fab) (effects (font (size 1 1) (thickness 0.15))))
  (pad 1 smd rect (at -0.75 0) (size 0.5 0.9) (layers F.Cu F.Paste F.Mask) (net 63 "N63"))
  (pad 2 smd rect (at 0.75 0) (size 0.5 0.9) (layers F.Cu F.Paste F.Mask) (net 17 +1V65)))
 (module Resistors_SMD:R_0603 (layer F.Cu) (at 196.977 98.044)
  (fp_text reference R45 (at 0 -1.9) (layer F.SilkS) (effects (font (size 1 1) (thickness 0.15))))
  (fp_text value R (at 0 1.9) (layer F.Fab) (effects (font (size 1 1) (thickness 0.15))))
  (pad 1 smd rect (at -0.75 0) (size 0.5 0.9) (layers F.Cu F.Paste F.Mask) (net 81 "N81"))
  (pad 2 smd rect (at 0.75 0) (size 0.5 0.9) (layers F.Cu F.Paste F.Mask) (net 82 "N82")))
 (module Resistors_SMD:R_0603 (layer F.Cu) (at 200.787 98.044)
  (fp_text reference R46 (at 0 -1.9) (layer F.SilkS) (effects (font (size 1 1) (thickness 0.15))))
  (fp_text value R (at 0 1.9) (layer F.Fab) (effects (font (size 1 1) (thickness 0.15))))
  (pad 1 smd rect (at -0.75 0) (size 0.5 0.9) (layers F.Cu F.Paste F.Mask) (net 82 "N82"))
  (pad 2 smd rect (at 0.75 0) (size 0.5 0.9) (layers F.Cu F.Paste F.Mask) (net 17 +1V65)))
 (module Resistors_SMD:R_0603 (layer F.Cu) (at 201.803 101.092)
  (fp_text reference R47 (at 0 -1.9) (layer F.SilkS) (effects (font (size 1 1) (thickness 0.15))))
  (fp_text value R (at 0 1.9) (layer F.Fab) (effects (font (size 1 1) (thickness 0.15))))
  (pad 1 smd rect (at -0.75 0) (size 0.5 0.9) (layers F.Cu F.Paste F.Mask) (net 83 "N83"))
  (pad 2 smd rect (at 0.75 0) (size 0.5 0.9) (layers F.Cu F.Paste F.Mask) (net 84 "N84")))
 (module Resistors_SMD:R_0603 (layer F.Cu) (at 201.803 103.886)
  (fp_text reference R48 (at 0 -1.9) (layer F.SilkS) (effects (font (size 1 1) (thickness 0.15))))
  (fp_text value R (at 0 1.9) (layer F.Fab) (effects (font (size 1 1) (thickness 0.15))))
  (pad 1 smd rect (at -0.75 0) (size 0.5 0.9) (layers F.Cu F.Paste F.Mask) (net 84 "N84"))
  (pad 2 smd rect (at 0.75 0) (size 0.5 0.9) (layers F.Cu F.Paste F.Mask) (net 17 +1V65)))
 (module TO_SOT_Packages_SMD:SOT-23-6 (layer F.Cu) (at 197.231 108.458)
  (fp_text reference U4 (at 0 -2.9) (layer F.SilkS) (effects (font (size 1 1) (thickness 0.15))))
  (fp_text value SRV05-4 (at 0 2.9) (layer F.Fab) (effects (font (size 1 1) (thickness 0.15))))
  (pad 1 smd rect (at -1.1 -0.95) (size 1.06 0.65) (layers F.Cu F.Paste F.Mask) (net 64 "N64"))
  (pad 2 smd rect (at -1.1 0) (size 1.06 0.65) (layers F.Cu F.Paste F.Mask) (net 4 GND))
  (pad 3 smd rect (at -1.1 0.95) (size 1.06 0.65) (layers F.Cu F.Paste F.Mask) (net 63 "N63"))
  (pad 4 smd rect (at 1.1 0.95) (size 1.06 0.65) (layers F.Cu F.Paste F.Mask) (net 60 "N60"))
  (pad 6 smd rect (at 1.1 -0.95) (size 1.06 0.65) (layers F.Cu F.Paste F.Mask) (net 62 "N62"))
  (pad 5 smd rect (at 1.1 0) (size 1.06 0.65) (layers F.Cu F.Paste F.Mask) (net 80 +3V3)))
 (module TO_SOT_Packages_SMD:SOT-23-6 (layer F.Cu) (at 194.945 114.3)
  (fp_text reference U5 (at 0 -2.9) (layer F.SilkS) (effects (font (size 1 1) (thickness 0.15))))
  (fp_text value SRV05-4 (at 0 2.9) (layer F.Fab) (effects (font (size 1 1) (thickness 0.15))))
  (pad 1 smd rect (at -1.1 -0.95) (size 1.06 0.65) (layers F.Cu F.Paste F.Mask) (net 83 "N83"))
  (pad 2 smd rect (at -1.1 0) (size 1.06 0.65) (layers F.Cu F.Paste F.Mask) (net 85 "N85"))
  (pad 3 smd rect (at -1.1 0.95) (size 1.06 0.65) (layers F.Cu F.Paste F.Mask) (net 84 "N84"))
  (pad 4 smd rect (at 1.1 0.95) (size 1.06 0.65) (layers F.Cu F.Paste F.Mask) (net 82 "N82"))
  (pad 6 smd rect (at 1.1 -0.95) (size 1.06 0.65) (layers F.Cu F.Paste F.Mask) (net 81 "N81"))
  (pad 5 smd rect (at 1.1 0) (size 1.06 0.65) (layers F.Cu F.Paste F.Mask) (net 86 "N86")))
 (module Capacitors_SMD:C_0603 (layer F.Cu) (at 191.123 110.617)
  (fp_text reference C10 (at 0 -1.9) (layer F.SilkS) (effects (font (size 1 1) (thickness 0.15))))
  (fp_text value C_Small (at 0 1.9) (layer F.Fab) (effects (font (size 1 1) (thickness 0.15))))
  (pad 1 smd rect (at -0.75 0) (size 0.8 0.75) (layers F.Cu F.Paste F.Mask) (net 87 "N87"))
  (pad 2 smd rect (at 0.75 0) (size 0.8 0.75) (layers F.Cu F.Paste F.Mask) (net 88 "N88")))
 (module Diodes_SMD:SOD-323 (layer F.Cu) (at 206.883 111.379)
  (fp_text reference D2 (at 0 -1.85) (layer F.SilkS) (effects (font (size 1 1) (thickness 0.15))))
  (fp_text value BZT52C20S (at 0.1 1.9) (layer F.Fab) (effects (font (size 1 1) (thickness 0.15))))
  (pad 1 smd rect (at -1.055 0) (size 0.59 0.45) (layers F.Cu F.Paste F.Mask) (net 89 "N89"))
  (pad 2 smd rect (at 1.055 0) (size 0.59 0.45) (layers F.Cu F.Paste F.Mask) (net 87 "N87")))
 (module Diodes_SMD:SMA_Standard (layer F.Cu) (at 200.914 114.808)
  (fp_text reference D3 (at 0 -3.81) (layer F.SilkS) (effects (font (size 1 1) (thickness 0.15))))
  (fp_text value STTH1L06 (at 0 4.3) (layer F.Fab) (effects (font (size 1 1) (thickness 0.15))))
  (pad 1 smd rect (at -1.99898 0) (size 2.49936 1.80086) (layers F.Cu F.Paste F.Mask) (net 89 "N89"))
  (pad 2 smd rect (at 1.99898 0) (size 2.49936 1.80086) (layers F.Cu F.Paste F.Mask) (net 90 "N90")))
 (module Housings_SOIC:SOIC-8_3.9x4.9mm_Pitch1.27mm (layer F.Cu) (at 196.85 103.928001)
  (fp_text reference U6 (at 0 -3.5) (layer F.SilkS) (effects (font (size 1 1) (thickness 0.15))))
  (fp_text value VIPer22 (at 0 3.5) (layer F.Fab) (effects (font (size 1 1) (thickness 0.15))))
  (pad 1 smd rect (at -2.7 -1.905) (size 1.55 0.6) (layers F.Cu F.Paste F.Mask) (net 88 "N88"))
  (pad 2 smd rect (at -2.7 -0.635) (size 1.55 0.6) (layers F.Cu F.Paste F.Mask) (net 88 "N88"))
  (pad 3 smd rect (at -2.7 0.635) (size 1.55 0.6) (layers F.Cu F.Paste F.Mask) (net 87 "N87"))
  (pad 4 smd rect (at -2.7 1.905) (size 1.55 0.6) (layers F.Cu F.Paste F.Mask) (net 89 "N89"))
  (pad 5 smd rect (at 2.7 1.905) (size 1.55 0.6) (layers F.Cu F.Paste F.Mask) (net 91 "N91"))
  (pad 6 smd rect (at 2.7 0.635) (size 1.55 0.6) (layers F.Cu F.Paste F.Mask) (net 91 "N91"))
  (pad 7 smd rect (at 2.7 -0.635) (size 1.55 0.6) (layers F.Cu F.Paste F.Mask) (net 91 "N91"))
  (pad 8 smd rect (at 2.7 -1.905) (size 1.55 0.6) (layers F.Cu F.Paste F.Mask) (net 91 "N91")))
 (gr_line (start 135.89 45.593) (end 135.89 46.863) (angle 90) (layer Edge.Cuts) (width 0.15))
 (gr_line (start 257.81 45.593) (end 135.89 45.593) (angle 90) (layer Edge.Cuts) (width 0.15))
 (gr_line (start 257.81 93.853) (end 257.81 45.593) (angle 90) (layer Edge.Cuts) (width 0.15))
 (gr_line (start 135.89 93.98) (end 257.81 93.853) (angle 90) (layer Edge.Cuts) (width 0.15))
 (gr_line (start 135.89 46.863) (end 135.89 93.98) (angle 90) (layer Edge.Cuts) (width 0.15))
 (segment (start 218.567 43.295) (end 218.567 47.879) (width 0.25) (layer F.Cu) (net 12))
 (segment (start 218.821 48.133) (end 220.82 48.133) (width 0.25) (layer F.Cu) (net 12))
 (segment (start 218.567 47.879) (end 218.821 48.133) (width 0.25) (layer F.Cu) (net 12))
 (segment (start 220.82 41.783) (end 218.579 41.783) (width 0.25) (layer F.Cu) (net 13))
 (segment (start 218.579 41.783) (end 218.567 41.795) (width 0.25) (layer F.Cu) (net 13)))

